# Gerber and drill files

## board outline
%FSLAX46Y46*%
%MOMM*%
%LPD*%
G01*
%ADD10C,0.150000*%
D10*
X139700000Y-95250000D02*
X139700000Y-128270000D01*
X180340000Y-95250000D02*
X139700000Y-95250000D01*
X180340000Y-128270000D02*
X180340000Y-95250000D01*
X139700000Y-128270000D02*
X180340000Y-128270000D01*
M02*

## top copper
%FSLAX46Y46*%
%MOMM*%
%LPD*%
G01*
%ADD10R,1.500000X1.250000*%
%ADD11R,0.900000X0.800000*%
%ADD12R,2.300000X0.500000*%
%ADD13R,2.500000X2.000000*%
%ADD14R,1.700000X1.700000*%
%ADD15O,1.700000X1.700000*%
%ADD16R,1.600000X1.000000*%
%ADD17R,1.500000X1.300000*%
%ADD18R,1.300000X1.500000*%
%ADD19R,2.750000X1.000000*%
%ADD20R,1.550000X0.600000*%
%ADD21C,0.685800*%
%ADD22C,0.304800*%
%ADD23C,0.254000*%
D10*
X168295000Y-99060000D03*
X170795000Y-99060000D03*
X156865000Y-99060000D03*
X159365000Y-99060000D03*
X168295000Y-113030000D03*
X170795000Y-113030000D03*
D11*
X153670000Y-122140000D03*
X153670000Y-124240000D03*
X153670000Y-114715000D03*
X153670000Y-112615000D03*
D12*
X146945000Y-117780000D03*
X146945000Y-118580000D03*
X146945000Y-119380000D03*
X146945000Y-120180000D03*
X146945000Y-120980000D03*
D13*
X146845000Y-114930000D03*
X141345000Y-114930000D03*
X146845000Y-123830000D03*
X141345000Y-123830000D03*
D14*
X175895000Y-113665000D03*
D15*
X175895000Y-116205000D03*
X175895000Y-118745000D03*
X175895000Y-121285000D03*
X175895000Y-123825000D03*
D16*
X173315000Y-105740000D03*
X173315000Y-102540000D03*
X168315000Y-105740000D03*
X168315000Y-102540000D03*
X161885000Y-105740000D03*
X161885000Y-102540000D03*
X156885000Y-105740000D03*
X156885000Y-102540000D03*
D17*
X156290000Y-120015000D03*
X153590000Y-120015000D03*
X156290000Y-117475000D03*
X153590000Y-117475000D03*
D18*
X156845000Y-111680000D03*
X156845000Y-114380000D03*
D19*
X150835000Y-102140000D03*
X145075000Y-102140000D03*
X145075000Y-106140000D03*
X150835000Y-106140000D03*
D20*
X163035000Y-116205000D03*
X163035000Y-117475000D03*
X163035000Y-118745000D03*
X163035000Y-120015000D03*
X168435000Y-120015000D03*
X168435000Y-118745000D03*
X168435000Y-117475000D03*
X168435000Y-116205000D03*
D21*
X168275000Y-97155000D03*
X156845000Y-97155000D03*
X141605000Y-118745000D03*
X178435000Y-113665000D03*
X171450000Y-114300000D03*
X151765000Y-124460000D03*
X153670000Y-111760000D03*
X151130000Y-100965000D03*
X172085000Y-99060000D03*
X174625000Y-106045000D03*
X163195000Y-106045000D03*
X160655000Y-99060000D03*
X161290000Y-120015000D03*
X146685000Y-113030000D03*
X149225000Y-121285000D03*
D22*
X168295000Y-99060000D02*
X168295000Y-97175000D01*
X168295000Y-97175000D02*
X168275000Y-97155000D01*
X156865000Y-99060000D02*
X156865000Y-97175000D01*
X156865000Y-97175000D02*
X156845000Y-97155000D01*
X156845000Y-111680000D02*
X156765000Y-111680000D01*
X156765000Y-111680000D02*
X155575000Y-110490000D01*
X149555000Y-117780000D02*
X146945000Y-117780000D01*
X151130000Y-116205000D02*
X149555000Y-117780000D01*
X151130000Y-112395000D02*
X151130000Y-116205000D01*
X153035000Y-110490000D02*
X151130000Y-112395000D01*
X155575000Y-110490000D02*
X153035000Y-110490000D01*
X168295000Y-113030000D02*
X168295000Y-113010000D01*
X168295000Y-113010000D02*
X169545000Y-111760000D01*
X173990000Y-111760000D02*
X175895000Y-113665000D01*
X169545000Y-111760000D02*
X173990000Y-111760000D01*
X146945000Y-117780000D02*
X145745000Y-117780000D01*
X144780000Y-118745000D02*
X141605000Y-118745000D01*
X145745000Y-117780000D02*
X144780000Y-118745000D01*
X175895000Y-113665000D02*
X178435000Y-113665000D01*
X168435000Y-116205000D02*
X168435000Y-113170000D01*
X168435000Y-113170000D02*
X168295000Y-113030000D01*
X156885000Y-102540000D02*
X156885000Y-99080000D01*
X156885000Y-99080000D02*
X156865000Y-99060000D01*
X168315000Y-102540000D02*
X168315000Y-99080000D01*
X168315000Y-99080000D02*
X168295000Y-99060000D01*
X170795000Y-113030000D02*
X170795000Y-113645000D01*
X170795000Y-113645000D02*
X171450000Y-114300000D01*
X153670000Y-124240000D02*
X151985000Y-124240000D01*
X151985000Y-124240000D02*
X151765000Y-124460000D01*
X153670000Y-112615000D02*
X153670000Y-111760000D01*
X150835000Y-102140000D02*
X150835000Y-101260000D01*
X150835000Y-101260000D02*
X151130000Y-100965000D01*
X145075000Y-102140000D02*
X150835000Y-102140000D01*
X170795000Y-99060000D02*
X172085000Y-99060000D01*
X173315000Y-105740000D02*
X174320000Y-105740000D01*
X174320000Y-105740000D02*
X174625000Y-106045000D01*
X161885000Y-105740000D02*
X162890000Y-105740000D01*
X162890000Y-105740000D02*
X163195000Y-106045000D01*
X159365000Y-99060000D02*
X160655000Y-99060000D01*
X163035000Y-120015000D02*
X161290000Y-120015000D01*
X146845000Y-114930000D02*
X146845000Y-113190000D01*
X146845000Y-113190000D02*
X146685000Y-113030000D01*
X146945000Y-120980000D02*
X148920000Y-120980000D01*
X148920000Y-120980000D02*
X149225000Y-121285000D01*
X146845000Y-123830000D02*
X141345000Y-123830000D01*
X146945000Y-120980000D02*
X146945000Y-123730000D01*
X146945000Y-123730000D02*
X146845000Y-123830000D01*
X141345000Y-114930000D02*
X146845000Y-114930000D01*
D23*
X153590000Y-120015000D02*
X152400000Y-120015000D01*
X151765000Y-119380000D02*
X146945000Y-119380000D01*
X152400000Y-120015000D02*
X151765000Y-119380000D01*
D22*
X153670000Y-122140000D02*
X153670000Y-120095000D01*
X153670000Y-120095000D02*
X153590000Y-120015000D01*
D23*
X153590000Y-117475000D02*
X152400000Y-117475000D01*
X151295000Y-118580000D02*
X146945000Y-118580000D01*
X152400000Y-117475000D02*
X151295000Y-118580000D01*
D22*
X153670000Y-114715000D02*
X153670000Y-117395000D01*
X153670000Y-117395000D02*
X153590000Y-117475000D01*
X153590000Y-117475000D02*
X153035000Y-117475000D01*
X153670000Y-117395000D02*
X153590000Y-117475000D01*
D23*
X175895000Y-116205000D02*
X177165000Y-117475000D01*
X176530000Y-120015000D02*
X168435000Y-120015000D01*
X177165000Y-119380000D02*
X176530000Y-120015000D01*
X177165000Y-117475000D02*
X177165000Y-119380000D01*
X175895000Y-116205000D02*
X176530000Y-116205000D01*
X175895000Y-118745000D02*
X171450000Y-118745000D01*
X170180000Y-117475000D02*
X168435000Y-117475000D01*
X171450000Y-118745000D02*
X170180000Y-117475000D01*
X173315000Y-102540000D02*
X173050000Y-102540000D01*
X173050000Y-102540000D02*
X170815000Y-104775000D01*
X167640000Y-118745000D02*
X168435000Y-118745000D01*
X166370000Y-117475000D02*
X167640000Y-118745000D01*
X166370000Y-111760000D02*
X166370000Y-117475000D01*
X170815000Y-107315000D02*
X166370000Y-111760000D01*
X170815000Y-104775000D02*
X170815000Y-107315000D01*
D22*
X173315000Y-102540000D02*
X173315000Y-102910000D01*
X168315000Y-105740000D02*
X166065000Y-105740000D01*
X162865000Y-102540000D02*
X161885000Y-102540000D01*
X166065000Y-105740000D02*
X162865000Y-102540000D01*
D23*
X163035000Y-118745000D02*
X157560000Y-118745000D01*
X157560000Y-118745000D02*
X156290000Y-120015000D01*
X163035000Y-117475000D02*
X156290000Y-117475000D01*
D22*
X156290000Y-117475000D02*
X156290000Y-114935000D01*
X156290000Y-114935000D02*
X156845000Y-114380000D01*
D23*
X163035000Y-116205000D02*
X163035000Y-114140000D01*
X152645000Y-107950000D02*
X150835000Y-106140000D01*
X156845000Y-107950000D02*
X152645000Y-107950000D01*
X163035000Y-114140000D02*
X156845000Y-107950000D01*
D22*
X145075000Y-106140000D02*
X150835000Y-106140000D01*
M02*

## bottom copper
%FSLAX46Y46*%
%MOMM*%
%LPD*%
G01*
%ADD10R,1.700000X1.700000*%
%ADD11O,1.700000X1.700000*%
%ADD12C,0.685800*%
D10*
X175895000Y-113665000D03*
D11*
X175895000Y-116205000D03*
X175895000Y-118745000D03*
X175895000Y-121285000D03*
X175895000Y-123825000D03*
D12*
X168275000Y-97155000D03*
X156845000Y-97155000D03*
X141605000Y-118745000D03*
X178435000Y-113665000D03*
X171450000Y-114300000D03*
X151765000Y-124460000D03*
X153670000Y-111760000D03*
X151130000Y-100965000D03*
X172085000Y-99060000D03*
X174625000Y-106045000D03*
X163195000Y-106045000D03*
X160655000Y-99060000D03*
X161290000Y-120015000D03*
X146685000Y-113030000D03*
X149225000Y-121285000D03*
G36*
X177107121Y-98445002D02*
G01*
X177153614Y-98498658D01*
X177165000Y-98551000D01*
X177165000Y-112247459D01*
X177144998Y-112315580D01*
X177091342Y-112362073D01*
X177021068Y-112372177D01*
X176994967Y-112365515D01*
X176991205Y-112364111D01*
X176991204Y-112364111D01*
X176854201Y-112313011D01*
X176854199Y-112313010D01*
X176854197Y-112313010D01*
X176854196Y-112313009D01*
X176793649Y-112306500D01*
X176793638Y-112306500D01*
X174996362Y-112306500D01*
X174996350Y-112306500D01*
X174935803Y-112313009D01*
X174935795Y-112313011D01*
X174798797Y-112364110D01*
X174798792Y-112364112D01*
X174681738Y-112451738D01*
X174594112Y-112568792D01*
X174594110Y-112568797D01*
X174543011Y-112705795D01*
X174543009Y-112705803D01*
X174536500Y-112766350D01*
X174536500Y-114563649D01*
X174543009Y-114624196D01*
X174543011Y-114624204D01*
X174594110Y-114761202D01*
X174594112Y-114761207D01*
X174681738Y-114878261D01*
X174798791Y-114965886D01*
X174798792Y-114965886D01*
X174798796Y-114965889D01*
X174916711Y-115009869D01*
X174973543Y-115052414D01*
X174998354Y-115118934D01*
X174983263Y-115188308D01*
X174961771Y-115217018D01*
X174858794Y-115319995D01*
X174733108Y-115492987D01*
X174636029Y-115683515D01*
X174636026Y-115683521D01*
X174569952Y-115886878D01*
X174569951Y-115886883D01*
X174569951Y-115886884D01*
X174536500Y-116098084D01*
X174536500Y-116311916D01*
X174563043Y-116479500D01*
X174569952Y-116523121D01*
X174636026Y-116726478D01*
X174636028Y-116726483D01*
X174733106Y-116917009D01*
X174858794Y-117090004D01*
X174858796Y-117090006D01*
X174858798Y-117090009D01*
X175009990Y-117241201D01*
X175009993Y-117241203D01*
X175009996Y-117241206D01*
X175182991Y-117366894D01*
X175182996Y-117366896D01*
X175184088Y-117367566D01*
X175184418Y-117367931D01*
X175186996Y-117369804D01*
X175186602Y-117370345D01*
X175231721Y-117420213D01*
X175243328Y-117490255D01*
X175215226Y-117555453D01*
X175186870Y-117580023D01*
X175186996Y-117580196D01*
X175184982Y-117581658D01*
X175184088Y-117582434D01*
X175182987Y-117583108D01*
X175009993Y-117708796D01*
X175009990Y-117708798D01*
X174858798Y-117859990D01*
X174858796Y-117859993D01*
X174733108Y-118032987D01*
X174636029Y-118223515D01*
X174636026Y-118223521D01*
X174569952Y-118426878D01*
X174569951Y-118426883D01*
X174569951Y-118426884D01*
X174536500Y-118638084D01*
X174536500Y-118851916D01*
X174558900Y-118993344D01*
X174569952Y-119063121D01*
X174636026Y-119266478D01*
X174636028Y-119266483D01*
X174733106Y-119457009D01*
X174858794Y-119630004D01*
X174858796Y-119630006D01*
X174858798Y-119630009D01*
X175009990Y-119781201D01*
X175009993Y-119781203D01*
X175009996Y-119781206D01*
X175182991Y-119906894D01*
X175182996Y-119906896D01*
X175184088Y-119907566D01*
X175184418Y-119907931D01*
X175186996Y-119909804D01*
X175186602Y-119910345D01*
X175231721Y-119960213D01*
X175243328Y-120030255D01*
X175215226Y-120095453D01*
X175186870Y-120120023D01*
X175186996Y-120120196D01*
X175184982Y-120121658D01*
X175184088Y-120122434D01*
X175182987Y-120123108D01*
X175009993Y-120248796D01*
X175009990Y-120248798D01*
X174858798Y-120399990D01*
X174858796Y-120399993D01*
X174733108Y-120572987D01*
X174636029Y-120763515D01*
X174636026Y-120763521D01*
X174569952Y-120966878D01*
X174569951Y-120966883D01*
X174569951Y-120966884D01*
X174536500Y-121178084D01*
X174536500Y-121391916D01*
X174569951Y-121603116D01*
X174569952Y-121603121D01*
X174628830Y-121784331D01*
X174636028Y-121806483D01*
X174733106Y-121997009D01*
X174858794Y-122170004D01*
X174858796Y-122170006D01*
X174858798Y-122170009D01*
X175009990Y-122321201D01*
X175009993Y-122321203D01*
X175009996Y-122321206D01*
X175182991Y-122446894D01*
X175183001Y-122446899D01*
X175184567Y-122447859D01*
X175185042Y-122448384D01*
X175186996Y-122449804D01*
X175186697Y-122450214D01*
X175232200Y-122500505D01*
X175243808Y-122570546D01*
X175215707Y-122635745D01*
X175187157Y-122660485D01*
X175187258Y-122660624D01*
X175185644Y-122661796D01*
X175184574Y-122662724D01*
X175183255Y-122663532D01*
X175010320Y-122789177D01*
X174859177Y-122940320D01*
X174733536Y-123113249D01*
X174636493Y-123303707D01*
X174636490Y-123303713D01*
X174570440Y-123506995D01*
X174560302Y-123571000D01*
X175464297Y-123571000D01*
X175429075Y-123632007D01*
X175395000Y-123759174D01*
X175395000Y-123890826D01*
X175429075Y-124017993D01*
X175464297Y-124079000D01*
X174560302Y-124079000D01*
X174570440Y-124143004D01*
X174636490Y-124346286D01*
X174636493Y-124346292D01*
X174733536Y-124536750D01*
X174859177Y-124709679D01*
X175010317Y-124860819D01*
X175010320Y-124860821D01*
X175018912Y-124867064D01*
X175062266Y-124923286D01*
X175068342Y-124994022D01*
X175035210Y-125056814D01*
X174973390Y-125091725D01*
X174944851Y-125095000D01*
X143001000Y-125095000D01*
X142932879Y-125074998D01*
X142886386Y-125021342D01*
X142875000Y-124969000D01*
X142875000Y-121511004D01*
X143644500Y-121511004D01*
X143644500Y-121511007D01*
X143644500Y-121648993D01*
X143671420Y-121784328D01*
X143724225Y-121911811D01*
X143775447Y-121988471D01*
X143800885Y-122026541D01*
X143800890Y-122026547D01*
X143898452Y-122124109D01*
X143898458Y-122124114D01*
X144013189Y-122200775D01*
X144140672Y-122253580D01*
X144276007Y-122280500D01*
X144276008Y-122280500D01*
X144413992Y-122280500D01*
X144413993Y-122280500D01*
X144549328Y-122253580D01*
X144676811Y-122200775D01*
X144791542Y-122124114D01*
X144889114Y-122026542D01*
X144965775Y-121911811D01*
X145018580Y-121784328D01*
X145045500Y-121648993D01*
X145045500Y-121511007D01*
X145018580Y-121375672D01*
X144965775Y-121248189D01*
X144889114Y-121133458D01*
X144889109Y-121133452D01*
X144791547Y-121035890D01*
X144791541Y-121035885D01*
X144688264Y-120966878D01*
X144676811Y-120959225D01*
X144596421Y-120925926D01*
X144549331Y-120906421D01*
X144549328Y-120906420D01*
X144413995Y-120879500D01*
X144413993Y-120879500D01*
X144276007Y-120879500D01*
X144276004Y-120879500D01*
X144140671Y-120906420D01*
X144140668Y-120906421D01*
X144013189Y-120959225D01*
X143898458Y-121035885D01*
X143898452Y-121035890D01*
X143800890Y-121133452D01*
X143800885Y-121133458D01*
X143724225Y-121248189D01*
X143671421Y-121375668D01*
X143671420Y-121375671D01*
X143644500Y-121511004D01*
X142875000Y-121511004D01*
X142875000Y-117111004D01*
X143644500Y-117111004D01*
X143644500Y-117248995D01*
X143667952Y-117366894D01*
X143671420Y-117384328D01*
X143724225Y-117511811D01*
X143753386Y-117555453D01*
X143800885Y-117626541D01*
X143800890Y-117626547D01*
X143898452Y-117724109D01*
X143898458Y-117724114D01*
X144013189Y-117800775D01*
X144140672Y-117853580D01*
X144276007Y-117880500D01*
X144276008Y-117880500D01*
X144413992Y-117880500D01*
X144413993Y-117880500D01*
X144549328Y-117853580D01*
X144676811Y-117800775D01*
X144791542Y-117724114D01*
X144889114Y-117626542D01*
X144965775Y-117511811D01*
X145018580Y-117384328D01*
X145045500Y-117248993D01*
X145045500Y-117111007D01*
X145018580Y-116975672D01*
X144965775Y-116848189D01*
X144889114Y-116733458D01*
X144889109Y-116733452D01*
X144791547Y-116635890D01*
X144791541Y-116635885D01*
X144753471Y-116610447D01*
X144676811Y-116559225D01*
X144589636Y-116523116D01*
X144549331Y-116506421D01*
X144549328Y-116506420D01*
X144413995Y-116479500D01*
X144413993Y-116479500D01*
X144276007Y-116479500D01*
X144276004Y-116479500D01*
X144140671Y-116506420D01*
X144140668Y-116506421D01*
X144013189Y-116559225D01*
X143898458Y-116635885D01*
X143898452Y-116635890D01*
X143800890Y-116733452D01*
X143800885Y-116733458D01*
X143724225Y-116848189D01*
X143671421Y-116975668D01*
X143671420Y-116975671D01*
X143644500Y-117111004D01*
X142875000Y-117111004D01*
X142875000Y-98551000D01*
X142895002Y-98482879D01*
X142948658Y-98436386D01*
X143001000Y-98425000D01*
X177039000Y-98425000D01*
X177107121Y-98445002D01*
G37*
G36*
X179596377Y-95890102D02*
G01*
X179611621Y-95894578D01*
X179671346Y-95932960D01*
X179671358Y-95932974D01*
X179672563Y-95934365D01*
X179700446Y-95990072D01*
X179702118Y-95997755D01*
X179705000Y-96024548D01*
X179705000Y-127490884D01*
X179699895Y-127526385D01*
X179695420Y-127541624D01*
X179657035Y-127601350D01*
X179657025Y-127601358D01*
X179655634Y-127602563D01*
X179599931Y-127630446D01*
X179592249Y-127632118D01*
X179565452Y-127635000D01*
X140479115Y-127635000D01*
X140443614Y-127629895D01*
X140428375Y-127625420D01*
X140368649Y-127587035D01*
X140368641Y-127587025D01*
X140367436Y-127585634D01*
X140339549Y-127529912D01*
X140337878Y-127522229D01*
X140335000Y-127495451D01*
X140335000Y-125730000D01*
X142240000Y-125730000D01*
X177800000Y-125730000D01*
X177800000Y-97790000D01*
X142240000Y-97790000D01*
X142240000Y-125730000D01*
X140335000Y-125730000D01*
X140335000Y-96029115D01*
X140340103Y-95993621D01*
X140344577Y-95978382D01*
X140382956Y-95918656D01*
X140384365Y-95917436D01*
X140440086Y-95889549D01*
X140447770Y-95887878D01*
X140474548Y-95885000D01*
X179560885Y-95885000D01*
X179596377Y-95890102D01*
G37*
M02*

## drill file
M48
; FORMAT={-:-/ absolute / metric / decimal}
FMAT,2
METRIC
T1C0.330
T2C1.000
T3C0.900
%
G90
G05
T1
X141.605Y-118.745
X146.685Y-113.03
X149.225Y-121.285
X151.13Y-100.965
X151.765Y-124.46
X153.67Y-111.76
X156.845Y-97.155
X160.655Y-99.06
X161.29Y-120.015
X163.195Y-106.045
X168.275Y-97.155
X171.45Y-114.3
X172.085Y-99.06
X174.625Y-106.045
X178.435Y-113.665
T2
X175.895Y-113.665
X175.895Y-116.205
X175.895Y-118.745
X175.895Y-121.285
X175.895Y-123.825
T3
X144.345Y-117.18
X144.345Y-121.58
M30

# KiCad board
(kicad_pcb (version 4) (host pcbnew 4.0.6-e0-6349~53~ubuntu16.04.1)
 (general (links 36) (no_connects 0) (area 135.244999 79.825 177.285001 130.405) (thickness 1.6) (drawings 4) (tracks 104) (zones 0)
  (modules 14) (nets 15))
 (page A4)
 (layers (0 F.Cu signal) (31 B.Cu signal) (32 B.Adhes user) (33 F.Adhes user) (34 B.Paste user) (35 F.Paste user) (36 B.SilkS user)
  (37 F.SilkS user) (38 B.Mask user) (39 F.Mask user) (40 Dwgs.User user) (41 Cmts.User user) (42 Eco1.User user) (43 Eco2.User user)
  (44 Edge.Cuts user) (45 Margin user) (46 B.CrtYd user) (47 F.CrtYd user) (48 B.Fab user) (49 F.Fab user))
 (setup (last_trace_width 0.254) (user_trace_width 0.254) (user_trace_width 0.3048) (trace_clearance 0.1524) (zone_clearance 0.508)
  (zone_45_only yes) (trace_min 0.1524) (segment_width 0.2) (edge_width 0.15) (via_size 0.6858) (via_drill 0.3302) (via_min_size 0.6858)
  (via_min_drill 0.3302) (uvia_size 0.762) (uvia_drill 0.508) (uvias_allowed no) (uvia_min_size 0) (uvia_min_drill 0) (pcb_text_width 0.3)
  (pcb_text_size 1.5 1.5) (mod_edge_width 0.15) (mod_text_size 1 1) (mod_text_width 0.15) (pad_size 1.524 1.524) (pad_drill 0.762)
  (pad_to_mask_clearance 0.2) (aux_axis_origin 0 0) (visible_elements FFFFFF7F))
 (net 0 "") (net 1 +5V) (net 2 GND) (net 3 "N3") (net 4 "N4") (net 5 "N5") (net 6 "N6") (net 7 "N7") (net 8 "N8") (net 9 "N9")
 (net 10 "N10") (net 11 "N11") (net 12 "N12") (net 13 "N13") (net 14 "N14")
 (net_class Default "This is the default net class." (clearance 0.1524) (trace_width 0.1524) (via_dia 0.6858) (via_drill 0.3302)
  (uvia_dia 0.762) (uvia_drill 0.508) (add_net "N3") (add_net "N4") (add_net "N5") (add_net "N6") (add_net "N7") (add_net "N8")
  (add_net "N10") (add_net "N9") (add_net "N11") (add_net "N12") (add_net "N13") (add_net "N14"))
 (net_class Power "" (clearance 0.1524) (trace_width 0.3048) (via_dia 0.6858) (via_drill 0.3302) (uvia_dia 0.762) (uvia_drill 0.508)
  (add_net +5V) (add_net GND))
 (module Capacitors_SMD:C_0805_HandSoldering (layer F.Cu) (at 169.545 99.06)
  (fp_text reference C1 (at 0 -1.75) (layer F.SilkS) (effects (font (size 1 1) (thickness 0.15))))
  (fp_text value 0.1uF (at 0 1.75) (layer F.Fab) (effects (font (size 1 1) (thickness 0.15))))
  (pad 1 smd rect (at -1.25 0) (size 1.5 1.25) (layers F.Cu F.Paste F.Mask) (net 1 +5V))
  (pad 2 smd rect (at 1.25 0) (size 1.5 1.25) (layers F.Cu F.Paste F.Mask) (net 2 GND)))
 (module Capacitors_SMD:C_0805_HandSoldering (layer F.Cu) (at 158.115 99.06)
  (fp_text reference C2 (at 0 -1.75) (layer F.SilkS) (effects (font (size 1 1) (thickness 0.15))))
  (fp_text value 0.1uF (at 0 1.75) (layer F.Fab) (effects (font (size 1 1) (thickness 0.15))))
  (pad 1 smd rect (at -1.25 0) (size 1.5 1.25) (layers F.Cu F.Paste F.Mask) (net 1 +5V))
  (pad 2 smd rect (at 1.25 0) (size 1.5 1.25) (layers F.Cu F.Paste F.Mask) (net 2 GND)))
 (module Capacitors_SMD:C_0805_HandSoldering (layer F.Cu) (at 169.545 113.03)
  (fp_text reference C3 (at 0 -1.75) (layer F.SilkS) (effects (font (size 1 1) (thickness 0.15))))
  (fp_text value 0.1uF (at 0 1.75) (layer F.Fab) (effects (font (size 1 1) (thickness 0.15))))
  (pad 1 smd rect (at -1.25 0) (size 1.5 1.25) (layers F.Cu F.Paste F.Mask) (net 1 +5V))
  (pad 2 smd rect (at 1.25 0) (size 1.5 1.25) (layers F.Cu F.Paste F.Mask) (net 2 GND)))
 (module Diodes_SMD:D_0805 (layer F.Cu) (at 153.67 123.19 270)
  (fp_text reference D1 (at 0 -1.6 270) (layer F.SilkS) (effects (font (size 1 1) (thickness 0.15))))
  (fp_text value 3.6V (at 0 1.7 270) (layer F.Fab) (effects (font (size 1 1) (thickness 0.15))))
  (pad 1 smd rect (at -1.05 0 270) (size 0.8 0.9) (layers F.Cu F.Paste F.Mask) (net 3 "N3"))
  (pad 2 smd rect (at 1.05 0 270) (size 0.8 0.9) (layers F.Cu F.Paste F.Mask) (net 2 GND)))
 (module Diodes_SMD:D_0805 (layer F.Cu) (at 153.67 113.665 90)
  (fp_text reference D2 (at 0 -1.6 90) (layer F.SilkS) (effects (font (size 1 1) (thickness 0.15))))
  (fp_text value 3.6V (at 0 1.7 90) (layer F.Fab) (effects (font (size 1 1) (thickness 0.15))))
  (pad 1 smd rect (at -1.05 0 90) (size 0.8 0.9) (layers F.Cu F.Paste F.Mask) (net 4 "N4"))
  (pad 2 smd rect (at 1.05 0 90) (size 0.8 0.9) (layers F.Cu F.Paste F.Mask) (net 2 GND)))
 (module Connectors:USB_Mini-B (layer F.Cu) (at 144.145 119.38)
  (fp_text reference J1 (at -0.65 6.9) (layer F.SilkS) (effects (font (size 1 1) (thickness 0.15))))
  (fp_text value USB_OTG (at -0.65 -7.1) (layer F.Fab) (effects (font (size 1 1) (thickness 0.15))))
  (pad 1 smd rect (at 2.8 -1.6) (size 2.3 0.5) (layers F.Cu F.Paste F.Mask) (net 1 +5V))
  (pad 2 smd rect (at 2.8 -0.8) (size 2.3 0.5) (layers F.Cu F.Paste F.Mask) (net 4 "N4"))
  (pad 3 smd rect (at 2.8 0) (size 2.3 0.5) (layers F.Cu F.Paste F.Mask) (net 3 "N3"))
  (pad 4 smd rect (at 2.8 0.8) (size 2.3 0.5) (layers F.Cu F.Paste F.Mask) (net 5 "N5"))
  (pad 5 smd rect (at 2.8 1.6) (size 2.3 0.5) (layers F.Cu F.Paste F.Mask) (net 2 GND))
  (pad 6 smd rect (at 2.7 -4.45) (size 2.5 2) (layers F.Cu F.Paste F.Mask) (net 2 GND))
  (pad 6 smd rect (at -2.8 -4.45) (size 2.5 2) (layers F.Cu F.Paste F.Mask) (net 2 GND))
  (pad 6 smd rect (at 2.7 4.45) (size 2.5 2) (layers F.Cu F.Paste F.Mask) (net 2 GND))
  (pad 6 smd rect (at -2.8 4.45) (size 2.5 2) (layers F.Cu F.Paste F.Mask) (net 2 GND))
  (pad "" np_thru_hole circle (at 0.2 -2.2) (size 0.9 0.9) (drill 0.9) (layers *.Cu *.Mask))
  (pad "" np_thru_hole circle (at 0.2 2.2) (size 0.9 0.9) (drill 0.9) (layers *.Cu *.Mask)))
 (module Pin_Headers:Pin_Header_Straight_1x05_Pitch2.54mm (layer F.Cu) (at 175.895 113.665)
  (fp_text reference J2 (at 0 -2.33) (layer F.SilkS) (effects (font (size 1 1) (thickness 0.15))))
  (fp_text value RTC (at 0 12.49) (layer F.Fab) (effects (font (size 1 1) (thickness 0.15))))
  (pad 1 thru_hole rect (at 0 0) (size 1.7 1.7) (drill 1) (layers *.Cu *.Mask) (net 1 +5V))
  (pad 2 thru_hole oval (at 0 2.54) (size 1.7 1.7) (drill 1) (layers *.Cu *.Mask) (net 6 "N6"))
  (pad 3 thru_hole oval (at 0 5.08) (size 1.7 1.7) (drill 1) (layers *.Cu *.Mask) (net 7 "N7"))
  (pad 4 thru_hole oval (at 0 7.62) (size 1.7 1.7) (drill 1) (layers *.Cu *.Mask) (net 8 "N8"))
  (pad 5 thru_hole oval (at 0 10.16) (size 1.7 1.7) (drill 1) (layers *.Cu *.Mask) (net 2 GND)))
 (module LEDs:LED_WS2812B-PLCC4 (layer F.Cu) (at 170.815 104.14)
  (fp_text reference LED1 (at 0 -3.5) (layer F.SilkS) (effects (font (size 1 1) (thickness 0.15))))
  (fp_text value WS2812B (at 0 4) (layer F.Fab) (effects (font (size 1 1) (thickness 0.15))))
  (pad 3 smd rect (at 2.5 1.6) (size 1.6 1) (layers F.Cu F.Paste F.Mask) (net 2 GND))
  (pad 4 smd rect (at 2.5 -1.6) (size 1.6 1) (layers F.Cu F.Paste F.Mask) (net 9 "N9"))
  (pad 2 smd rect (at -2.5 1.6) (size 1.6 1) (layers F.Cu F.Paste F.Mask) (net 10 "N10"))
  (pad 1 smd rect (at -2.5 -1.6) (size 1.6 1) (layers F.Cu F.Paste F.Mask) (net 1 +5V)))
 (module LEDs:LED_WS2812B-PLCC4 (layer F.Cu) (at 159.385 104.14)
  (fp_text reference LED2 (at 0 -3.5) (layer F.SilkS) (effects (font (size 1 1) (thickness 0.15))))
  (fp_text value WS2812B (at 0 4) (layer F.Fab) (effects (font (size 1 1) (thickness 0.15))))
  (pad 3 smd rect (at 2.5 1.6) (size 1.6 1) (layers F.Cu F.Paste F.Mask) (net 2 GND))
  (pad 4 smd rect (at 2.5 -1.6) (size 1.6 1) (layers F.Cu F.Paste F.Mask) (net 10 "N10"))
  (pad 2 smd rect (at -2.5 1.6) (size 1.6 1) (layers F.Cu F.Paste F.Mask) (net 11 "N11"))
  (pad 1 smd rect (at -2.5 -1.6) (size 1.6 1) (layers F.Cu F.Paste F.Mask) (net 1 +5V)))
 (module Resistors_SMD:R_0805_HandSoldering (layer F.Cu) (at 154.94 120.015 180)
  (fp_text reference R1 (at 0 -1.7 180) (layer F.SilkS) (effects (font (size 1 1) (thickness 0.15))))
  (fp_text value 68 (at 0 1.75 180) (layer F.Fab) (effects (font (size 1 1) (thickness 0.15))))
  (pad 1 smd rect (at -1.35 0 180) (size 1.5 1.3) (layers F.Cu F.Paste F.Mask) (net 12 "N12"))
  (pad 2 smd rect (at 1.35 0 180) (size 1.5 1.3) (layers F.Cu F.Paste F.Mask) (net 3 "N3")))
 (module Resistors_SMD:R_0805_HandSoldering (layer F.Cu) (at 154.94 117.475 180)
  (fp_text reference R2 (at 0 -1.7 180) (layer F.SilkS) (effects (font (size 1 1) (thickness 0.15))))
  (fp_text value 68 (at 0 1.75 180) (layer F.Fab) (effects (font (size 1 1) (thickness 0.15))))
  (pad 1 smd rect (at -1.35 0 180) (size 1.5 1.3) (layers F.Cu F.Paste F.Mask) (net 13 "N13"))
  (pad 2 smd rect (at 1.35 0 180) (size 1.5 1.3) (layers F.Cu F.Paste F.Mask) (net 4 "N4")))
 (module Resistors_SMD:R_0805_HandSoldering (layer F.Cu) (at 156.845 113.03 270)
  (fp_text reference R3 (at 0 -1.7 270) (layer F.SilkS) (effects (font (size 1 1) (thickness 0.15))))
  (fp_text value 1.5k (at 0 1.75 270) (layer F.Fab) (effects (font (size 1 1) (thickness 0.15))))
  (pad 1 smd rect (at -1.35 0 270) (size 1.5 1.3) (layers F.Cu F.Paste F.Mask) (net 1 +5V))
  (pad 2 smd rect (at 1.35 0 270) (size 1.5 1.3) (layers F.Cu F.Paste F.Mask) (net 13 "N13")))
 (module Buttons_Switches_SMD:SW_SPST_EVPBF (layer F.Cu) (at 147.955 104.14)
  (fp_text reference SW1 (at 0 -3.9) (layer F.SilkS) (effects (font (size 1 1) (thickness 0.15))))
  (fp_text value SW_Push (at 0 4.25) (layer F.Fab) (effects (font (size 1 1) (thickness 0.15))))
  (pad 1 smd rect (at 2.88 -2) (size 2.75 1) (layers F.Cu F.Paste F.Mask) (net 2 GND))
  (pad 1 smd rect (at -2.88 -2) (size 2.75 1) (layers F.Cu F.Paste F.Mask) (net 2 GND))
  (pad 2 smd rect (at -2.88 2) (size 2.75 1) (layers F.Cu F.Paste F.Mask) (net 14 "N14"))
  (pad 2 smd rect (at 2.88 2) (size 2.75 1) (layers F.Cu F.Paste F.Mask) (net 14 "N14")))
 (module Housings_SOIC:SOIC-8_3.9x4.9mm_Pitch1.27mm (layer F.Cu) (at 165.735 118.11)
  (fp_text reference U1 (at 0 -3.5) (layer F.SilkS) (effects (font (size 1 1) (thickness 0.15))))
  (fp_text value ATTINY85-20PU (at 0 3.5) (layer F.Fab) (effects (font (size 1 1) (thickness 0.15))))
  (pad 1 smd rect (at -2.7 -1.905) (size 1.55 0.6) (layers F.Cu F.Paste F.Mask) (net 14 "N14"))
  (pad 2 smd rect (at -2.7 -0.635) (size 1.55 0.6) (layers F.Cu F.Paste F.Mask) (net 13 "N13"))
  (pad 3 smd rect (at -2.7 0.635) (size 1.55 0.6) (layers F.Cu F.Paste F.Mask) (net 12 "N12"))
  (pad 4 smd rect (at -2.7 1.905) (size 1.55 0.6) (layers F.Cu F.Paste F.Mask) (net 2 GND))
  (pad 5 smd rect (at 2.7 1.905) (size 1.55 0.6) (layers F.Cu F.Paste F.Mask) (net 6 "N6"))
  (pad 6 smd rect (at 2.7 0.635) (size 1.55 0.6) (layers F.Cu F.Paste F.Mask) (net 9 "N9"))
  (pad 7 smd rect (at 2.7 -0.635) (size 1.55 0.6) (layers F.Cu F.Paste F.Mask) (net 7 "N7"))
  (pad 8 smd rect (at 2.7 -1.905) (size 1.55 0.6) (layers F.Cu F.Paste F.Mask) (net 1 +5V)))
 (gr_line (start 139.7 95.25) (end 139.7 128.27) (angle 90) (layer Edge.Cuts) (width 0.15))
 (gr_line (start 180.34 95.25) (end 139.7 95.25) (angle 90) (layer Edge.Cuts) (width 0.15))
 (gr_line (start 180.34 128.27) (end 180.34 95.25) (angle 90) (layer Edge.Cuts) (width 0.15))
 (gr_line (start 139.7 128.27) (end 180.34 128.27) (angle 90) (layer Edge.Cuts) (width 0.15))
 (segment (start 168.295 99.06) (end 168.295 97.175) (width 0.3048) (layer F.Cu) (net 1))
 (via (at 168.275 97.155) (size 0.6858) (drill 0.3302) (layers F.Cu B.Cu) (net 1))
 (segment (start 168.295 97.175) (end 168.275 97.155) (width 0.3048) (layer F.Cu) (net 1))
 (segment (start 156.865 99.06) (end 156.865 97.175) (width 0.3048) (layer F.Cu) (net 1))
 (via (at 156.845 97.155) (size 0.6858) (drill 0.3302) (layers F.Cu B.Cu) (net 1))
 (segment (start 156.865 97.175) (end 156.845 97.155) (width 0.3048) (layer F.Cu) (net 1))
 (segment (start 156.845 111.68) (end 156.765 111.68) (width 0.3048) (layer F.Cu) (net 1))
 (segment (start 156.765 111.68) (end 155.575 110.49) (width 0.3048) (layer F.Cu) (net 1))
 (segment (start 149.555 117.78) (end 146.945 117.78) (width 0.3048) (layer F.Cu) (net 1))
 (segment (start 151.13 116.205) (end 149.555 117.78) (width 0.3048) (layer F.Cu) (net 1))
 (segment (start 151.13 112.395) (end 151.13 116.205) (width 0.3048) (layer F.Cu) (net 1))
 (segment (start 153.035 110.49) (end 151.13 112.395) (width 0.3048) (layer F.Cu) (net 1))
 (segment (start 155.575 110.49) (end 153.035 110.49) (width 0.3048) (layer F.Cu) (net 1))
 (segment (start 168.295 113.03) (end 168.295 113.01) (width 0.3048) (layer F.Cu) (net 1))
 (segment (start 168.295 113.01) (end 169.545 111.76) (width 0.3048) (layer F.Cu) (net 1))
 (segment (start 173.99 111.76) (end 175.895 113.665) (width 0.3048) (layer F.Cu) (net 1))
 (segment (start 169.545 111.76) (end 173.99 111.76) (width 0.3048) (layer F.Cu) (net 1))
 (segment (start 146.945 117.78) (end 145.745 117.78) (width 0.3048) (layer F.Cu) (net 1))
 (via (at 141.605 118.745) (size 0.6858) (drill 0.3302) (layers F.Cu B.Cu) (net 1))
 (segment (start 144.78 118.745) (end 141.605 118.745) (width 0.3048) (layer F.Cu) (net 1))
 (segment (start 145.745 117.78) (end 144.78 118.745) (width 0.3048) (layer F.Cu) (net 1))
 (segment (start 175.895 113.665) (end 178.435 113.665) (width 0.3048) (layer F.Cu) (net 1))
 (via (at 178.435 113.665) (size 0.6858) (drill 0.3302) (layers F.Cu B.Cu) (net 1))
 (segment (start 168.435 116.205) (end 168.435 113.17) (width 0.3048) (layer F.Cu) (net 1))
 (segment (start 168.435 113.17) (end 168.295 113.03) (width 0.3048) (layer F.Cu) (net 1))
 (segment (start 156.885 102.54) (end 156.885 99.08) (width 0.3048) (layer F.Cu) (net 1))
 (segment (start 156.885 99.08) (end 156.865 99.06) (width 0.3048) (layer F.Cu) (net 1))
 (segment (start 168.315 102.54) (end 168.315 99.08) (width 0.3048) (layer F.Cu) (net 1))
 (segment (start 168.315 99.08) (end 168.295 99.06) (width 0.3048) (layer F.Cu) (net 1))
 (segment (start 170.795 113.03) (end 170.795 113.645) (width 0.3048) (layer F.Cu) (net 2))
 (segment (start 170.795 113.645) (end 171.45 114.3) (width 0.3048) (layer F.Cu) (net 2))
 (via (at 171.45 114.3) (size 0.6858) (drill 0.3302) (layers F.Cu B.Cu) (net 2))
 (segment (start 153.67 124.24) (end 151.985 124.24) (width 0.3048) (layer F.Cu) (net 2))
 (via (at 151.765 124.46) (size 0.6858) (drill 0.3302) (layers F.Cu B.Cu) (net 2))
 (segment (start 151.985 124.24) (end 151.765 124.46) (width 0.3048) (layer F.Cu) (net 2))
 (segment (start 153.67 112.615) (end 153.67 111.76) (width 0.3048) (layer F.Cu) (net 2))
 (via (at 153.67 111.76) (size 0.6858) (drill 0.3302) (layers F.Cu B.Cu) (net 2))
 (segment (start 150.835 102.14) (end 150.835 101.26) (width 0.3048) (layer F.Cu) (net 2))
 (via (at 151.13 100.965) (size 0.6858) (drill 0.3302) (layers F.Cu B.Cu) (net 2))
 (segment (start 150.835 101.26) (end 151.13 100.965) (width 0.3048) (layer F.Cu) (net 2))
 (segment (start 145.075 102.14) (end 150.835 102.14) (width 0.3048) (layer F.Cu) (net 2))
 (segment (start 170.795 99.06) (end 172.085 99.06) (width 0.3048) (layer F.Cu) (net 2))
 (via (at 172.085 99.06) (size 0.6858) (drill 0.3302) (layers F.Cu B.Cu) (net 2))
 (segment (start 173.315 105.74) (end 174.32 105.74) (width 0.3048) (layer F.Cu) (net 2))
 (via (at 174.625 106.045) (size 0.6858) (drill 0.3302) (layers F.Cu B.Cu) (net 2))
 (segment (start 174.32 105.74) (end 174.625 106.045) (width 0.3048) (layer F.Cu) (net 2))
 (segment (start 161.885 105.74) (end 162.89 105.74) (width 0.3048) (layer F.Cu) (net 2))
 (via (at 163.195 106.045) (size 0.6858) (drill 0.3302) (layers F.Cu B.Cu) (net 2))
 (segment (start 162.89 105.74) (end 163.195 106.045) (width 0.3048) (layer F.Cu) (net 2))
 (segment (start 159.365 99.06) (end 160.655 99.06) (width 0.3048) (layer F.Cu) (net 2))
 (via (at 160.655 99.06) (size 0.6858) (drill 0.3302) (layers F.Cu B.Cu) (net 2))
 (segment (start 163.035 120.015) (end 161.29 120.015) (width 0.3048) (layer F.Cu) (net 2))
 (via (at 161.29 120.015) (size 0.6858) (drill 0.3302) (layers F.Cu B.Cu) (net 2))
 (segment (start 146.845 114.93) (end 146.845 113.19) (width 0.3048) (layer F.Cu) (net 2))
 (via (at 146.685 113.03) (size 0.6858) (drill 0.3302) (layers F.Cu B.Cu) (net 2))
 (segment (start 146.845 113.19) (end 146.685 113.03) (width 0.3048) (layer F.Cu) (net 2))
 (segment (start 146.945 120.98) (end 148.92 120.98) (width 0.3048) (layer F.Cu) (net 2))
 (via (at 149.225 121.285) (size 0.6858) (drill 0.3302) (layers F.Cu B.Cu) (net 2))
 (segment (start 148.92 120.98) (end 149.225 121.285) (width 0.3048) (layer F.Cu) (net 2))
 (segment (start 146.845 123.83) (end 141.345 123.83) (width 0.3048) (layer F.Cu) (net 2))
 (segment (start 146.945 120.98) (end 146.945 123.73) (width 0.3048) (layer F.Cu) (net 2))
 (segment (start 146.945 123.73) (end 146.845 123.83) (width 0.3048) (layer F.Cu) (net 2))
 (segment (start 141.345 114.93) (end 146.845 114.93) (width 0.3048) (layer F.Cu) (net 2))
 (segment (start 153.59 120.015) (end 152.4 120.015) (width 0.254) (layer F.Cu) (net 3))
 (segment (start 151.765 119.38) (end 146.945 119.38) (width 0.254) (layer F.Cu) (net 3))
 (segment (start 152.4 120.015) (end 151.765 119.38) (width 0.254) (layer F.Cu) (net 3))
 (segment (start 153.67 122.14) (end 153.67 120.095) (width 0.3048) (layer F.Cu) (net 3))
 (segment (start 153.67 120.095) (end 153.59 120.015) (width 0.3048) (layer F.Cu) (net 3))
 (segment (start 153.59 117.475) (end 152.4 117.475) (width 0.254) (layer F.Cu) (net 4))
 (segment (start 151.295 118.58) (end 146.945 118.58) (width 0.254) (layer F.Cu) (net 4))
 (segment (start 152.4 117.475) (end 151.295 118.58) (width 0.254) (layer F.Cu) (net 4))
 (segment (start 153.67 114.715) (end 153.67 117.395) (width 0.3048) (layer F.Cu) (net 4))
 (segment (start 153.67 117.395) (end 153.59 117.475) (width 0.3048) (layer F.Cu) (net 4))
 (segment (start 153.59 117.475) (end 153.035 117.475) (width 0.3048) (layer F.Cu) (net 4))
 (segment (start 153.67 117.395) (end 153.59 117.475) (width 0.3048) (layer F.Cu) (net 4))
 (segment (start 175.895 116.205) (end 177.165 117.475) (width 0.254) (layer F.Cu) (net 6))
 (segment (start 176.53 120.015) (end 168.435 120.015) (width 0.254) (layer F.Cu) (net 6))
 (segment (start 177.165 119.38) (end 176.53 120.015) (width 0.254) (layer F.Cu) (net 6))
 (segment (start 177.165 117.475) (end 177.165 119.38) (width 0.254) (layer F.Cu) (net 6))
 (segment (start 175.895 116.205) (end 176.53 116.205) (width 0.254) (layer F.Cu) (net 6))
 (segment (start 175.895 118.745) (end 171.45 118.745) (width 0.254) (layer F.Cu) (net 7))
 (segment (start 170.18 117.475) (end 168.435 117.475) (width 0.254) (layer F.Cu) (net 7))
 (segment (start 171.45 118.745) (end 170.18 117.475) (width 0.254) (layer F.Cu) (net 7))
 (segment (start 173.315 102.54) (end 173.05 102.54) (width 0.254) (layer F.Cu) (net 9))
 (segment (start 173.05 102.54) (end 170.815 104.775) (width 0.254) (layer F.Cu) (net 9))
 (segment (start 167.64 118.745) (end 168.435 118.745) (width 0.254) (layer F.Cu) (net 9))
 (segment (start 166.37 117.475) (end 167.64 118.745) (width 0.254) (layer F.Cu) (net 9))
 (segment (start 166.37 111.76) (end 166.37 117.475) (width 0.254) (layer F.Cu) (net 9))
 (segment (start 170.815 107.315) (end 166.37 111.76) (width 0.254) (layer F.Cu) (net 9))
 (segment (start 170.815 104.775) (end 170.815 107.315) (width 0.254) (layer F.Cu) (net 9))
 (segment (start 173.315 102.54) (end 173.315 102.91) (width 0.3048) (layer F.Cu) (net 9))
 (segment (start 168.315 105.74) (end 166.065 105.74) (width 0.3048) (layer F.Cu) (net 10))
 (segment (start 162.865 102.54) (end 161.885 102.54) (width 0.3048) (layer F.Cu) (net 10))
 (segment (start 166.065 105.74) (end 162.865 102.54) (width 0.3048) (layer F.Cu) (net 10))
 (segment (start 163.035 118.745) (end 157.56 118.745) (width 0.254) (layer F.Cu) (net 12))
 (segment (start 157.56 118.745) (end 156.29 120.015) (width 0.254) (layer F.Cu) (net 12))
 (segment (start 163.035 117.475) (end 156.29 117.475) (width 0.254) (layer F.Cu) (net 13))
 (segment (start 156.29 117.475) (end 156.29 114.935) (width 0.3048) (layer F.Cu) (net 13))
 (segment (start 156.29 114.935) (end 156.845 114.38) (width 0.3048) (layer F.Cu) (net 13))
 (segment (start 163.035 116.205) (end 163.035 114.14) (width 0.254) (layer F.Cu) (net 14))
 (segment (start 152.645 107.95) (end 150.835 106.14) (width 0.254) (layer F.Cu) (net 14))
 (segment (start 156.845 107.95) (end 152.645 107.95) (width 0.254) (layer F.Cu) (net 14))
 (segment (start 163.035 114.14) (end 156.845 107.95) (width 0.254) (layer F.Cu) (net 14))
 (segment (start 145.075 106.14) (end 150.835 106.14) (width 0.3048) (layer F.Cu) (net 14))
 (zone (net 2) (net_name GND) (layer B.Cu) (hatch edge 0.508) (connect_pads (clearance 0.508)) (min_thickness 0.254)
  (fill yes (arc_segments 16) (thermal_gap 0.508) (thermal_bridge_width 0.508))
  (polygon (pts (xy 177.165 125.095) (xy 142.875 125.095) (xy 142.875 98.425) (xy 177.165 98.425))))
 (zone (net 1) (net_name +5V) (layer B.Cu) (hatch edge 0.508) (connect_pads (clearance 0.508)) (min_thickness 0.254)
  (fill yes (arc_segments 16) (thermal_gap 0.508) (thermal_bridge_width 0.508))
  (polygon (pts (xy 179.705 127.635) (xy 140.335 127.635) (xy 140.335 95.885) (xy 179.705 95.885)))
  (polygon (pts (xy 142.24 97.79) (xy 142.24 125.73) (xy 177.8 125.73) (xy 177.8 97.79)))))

